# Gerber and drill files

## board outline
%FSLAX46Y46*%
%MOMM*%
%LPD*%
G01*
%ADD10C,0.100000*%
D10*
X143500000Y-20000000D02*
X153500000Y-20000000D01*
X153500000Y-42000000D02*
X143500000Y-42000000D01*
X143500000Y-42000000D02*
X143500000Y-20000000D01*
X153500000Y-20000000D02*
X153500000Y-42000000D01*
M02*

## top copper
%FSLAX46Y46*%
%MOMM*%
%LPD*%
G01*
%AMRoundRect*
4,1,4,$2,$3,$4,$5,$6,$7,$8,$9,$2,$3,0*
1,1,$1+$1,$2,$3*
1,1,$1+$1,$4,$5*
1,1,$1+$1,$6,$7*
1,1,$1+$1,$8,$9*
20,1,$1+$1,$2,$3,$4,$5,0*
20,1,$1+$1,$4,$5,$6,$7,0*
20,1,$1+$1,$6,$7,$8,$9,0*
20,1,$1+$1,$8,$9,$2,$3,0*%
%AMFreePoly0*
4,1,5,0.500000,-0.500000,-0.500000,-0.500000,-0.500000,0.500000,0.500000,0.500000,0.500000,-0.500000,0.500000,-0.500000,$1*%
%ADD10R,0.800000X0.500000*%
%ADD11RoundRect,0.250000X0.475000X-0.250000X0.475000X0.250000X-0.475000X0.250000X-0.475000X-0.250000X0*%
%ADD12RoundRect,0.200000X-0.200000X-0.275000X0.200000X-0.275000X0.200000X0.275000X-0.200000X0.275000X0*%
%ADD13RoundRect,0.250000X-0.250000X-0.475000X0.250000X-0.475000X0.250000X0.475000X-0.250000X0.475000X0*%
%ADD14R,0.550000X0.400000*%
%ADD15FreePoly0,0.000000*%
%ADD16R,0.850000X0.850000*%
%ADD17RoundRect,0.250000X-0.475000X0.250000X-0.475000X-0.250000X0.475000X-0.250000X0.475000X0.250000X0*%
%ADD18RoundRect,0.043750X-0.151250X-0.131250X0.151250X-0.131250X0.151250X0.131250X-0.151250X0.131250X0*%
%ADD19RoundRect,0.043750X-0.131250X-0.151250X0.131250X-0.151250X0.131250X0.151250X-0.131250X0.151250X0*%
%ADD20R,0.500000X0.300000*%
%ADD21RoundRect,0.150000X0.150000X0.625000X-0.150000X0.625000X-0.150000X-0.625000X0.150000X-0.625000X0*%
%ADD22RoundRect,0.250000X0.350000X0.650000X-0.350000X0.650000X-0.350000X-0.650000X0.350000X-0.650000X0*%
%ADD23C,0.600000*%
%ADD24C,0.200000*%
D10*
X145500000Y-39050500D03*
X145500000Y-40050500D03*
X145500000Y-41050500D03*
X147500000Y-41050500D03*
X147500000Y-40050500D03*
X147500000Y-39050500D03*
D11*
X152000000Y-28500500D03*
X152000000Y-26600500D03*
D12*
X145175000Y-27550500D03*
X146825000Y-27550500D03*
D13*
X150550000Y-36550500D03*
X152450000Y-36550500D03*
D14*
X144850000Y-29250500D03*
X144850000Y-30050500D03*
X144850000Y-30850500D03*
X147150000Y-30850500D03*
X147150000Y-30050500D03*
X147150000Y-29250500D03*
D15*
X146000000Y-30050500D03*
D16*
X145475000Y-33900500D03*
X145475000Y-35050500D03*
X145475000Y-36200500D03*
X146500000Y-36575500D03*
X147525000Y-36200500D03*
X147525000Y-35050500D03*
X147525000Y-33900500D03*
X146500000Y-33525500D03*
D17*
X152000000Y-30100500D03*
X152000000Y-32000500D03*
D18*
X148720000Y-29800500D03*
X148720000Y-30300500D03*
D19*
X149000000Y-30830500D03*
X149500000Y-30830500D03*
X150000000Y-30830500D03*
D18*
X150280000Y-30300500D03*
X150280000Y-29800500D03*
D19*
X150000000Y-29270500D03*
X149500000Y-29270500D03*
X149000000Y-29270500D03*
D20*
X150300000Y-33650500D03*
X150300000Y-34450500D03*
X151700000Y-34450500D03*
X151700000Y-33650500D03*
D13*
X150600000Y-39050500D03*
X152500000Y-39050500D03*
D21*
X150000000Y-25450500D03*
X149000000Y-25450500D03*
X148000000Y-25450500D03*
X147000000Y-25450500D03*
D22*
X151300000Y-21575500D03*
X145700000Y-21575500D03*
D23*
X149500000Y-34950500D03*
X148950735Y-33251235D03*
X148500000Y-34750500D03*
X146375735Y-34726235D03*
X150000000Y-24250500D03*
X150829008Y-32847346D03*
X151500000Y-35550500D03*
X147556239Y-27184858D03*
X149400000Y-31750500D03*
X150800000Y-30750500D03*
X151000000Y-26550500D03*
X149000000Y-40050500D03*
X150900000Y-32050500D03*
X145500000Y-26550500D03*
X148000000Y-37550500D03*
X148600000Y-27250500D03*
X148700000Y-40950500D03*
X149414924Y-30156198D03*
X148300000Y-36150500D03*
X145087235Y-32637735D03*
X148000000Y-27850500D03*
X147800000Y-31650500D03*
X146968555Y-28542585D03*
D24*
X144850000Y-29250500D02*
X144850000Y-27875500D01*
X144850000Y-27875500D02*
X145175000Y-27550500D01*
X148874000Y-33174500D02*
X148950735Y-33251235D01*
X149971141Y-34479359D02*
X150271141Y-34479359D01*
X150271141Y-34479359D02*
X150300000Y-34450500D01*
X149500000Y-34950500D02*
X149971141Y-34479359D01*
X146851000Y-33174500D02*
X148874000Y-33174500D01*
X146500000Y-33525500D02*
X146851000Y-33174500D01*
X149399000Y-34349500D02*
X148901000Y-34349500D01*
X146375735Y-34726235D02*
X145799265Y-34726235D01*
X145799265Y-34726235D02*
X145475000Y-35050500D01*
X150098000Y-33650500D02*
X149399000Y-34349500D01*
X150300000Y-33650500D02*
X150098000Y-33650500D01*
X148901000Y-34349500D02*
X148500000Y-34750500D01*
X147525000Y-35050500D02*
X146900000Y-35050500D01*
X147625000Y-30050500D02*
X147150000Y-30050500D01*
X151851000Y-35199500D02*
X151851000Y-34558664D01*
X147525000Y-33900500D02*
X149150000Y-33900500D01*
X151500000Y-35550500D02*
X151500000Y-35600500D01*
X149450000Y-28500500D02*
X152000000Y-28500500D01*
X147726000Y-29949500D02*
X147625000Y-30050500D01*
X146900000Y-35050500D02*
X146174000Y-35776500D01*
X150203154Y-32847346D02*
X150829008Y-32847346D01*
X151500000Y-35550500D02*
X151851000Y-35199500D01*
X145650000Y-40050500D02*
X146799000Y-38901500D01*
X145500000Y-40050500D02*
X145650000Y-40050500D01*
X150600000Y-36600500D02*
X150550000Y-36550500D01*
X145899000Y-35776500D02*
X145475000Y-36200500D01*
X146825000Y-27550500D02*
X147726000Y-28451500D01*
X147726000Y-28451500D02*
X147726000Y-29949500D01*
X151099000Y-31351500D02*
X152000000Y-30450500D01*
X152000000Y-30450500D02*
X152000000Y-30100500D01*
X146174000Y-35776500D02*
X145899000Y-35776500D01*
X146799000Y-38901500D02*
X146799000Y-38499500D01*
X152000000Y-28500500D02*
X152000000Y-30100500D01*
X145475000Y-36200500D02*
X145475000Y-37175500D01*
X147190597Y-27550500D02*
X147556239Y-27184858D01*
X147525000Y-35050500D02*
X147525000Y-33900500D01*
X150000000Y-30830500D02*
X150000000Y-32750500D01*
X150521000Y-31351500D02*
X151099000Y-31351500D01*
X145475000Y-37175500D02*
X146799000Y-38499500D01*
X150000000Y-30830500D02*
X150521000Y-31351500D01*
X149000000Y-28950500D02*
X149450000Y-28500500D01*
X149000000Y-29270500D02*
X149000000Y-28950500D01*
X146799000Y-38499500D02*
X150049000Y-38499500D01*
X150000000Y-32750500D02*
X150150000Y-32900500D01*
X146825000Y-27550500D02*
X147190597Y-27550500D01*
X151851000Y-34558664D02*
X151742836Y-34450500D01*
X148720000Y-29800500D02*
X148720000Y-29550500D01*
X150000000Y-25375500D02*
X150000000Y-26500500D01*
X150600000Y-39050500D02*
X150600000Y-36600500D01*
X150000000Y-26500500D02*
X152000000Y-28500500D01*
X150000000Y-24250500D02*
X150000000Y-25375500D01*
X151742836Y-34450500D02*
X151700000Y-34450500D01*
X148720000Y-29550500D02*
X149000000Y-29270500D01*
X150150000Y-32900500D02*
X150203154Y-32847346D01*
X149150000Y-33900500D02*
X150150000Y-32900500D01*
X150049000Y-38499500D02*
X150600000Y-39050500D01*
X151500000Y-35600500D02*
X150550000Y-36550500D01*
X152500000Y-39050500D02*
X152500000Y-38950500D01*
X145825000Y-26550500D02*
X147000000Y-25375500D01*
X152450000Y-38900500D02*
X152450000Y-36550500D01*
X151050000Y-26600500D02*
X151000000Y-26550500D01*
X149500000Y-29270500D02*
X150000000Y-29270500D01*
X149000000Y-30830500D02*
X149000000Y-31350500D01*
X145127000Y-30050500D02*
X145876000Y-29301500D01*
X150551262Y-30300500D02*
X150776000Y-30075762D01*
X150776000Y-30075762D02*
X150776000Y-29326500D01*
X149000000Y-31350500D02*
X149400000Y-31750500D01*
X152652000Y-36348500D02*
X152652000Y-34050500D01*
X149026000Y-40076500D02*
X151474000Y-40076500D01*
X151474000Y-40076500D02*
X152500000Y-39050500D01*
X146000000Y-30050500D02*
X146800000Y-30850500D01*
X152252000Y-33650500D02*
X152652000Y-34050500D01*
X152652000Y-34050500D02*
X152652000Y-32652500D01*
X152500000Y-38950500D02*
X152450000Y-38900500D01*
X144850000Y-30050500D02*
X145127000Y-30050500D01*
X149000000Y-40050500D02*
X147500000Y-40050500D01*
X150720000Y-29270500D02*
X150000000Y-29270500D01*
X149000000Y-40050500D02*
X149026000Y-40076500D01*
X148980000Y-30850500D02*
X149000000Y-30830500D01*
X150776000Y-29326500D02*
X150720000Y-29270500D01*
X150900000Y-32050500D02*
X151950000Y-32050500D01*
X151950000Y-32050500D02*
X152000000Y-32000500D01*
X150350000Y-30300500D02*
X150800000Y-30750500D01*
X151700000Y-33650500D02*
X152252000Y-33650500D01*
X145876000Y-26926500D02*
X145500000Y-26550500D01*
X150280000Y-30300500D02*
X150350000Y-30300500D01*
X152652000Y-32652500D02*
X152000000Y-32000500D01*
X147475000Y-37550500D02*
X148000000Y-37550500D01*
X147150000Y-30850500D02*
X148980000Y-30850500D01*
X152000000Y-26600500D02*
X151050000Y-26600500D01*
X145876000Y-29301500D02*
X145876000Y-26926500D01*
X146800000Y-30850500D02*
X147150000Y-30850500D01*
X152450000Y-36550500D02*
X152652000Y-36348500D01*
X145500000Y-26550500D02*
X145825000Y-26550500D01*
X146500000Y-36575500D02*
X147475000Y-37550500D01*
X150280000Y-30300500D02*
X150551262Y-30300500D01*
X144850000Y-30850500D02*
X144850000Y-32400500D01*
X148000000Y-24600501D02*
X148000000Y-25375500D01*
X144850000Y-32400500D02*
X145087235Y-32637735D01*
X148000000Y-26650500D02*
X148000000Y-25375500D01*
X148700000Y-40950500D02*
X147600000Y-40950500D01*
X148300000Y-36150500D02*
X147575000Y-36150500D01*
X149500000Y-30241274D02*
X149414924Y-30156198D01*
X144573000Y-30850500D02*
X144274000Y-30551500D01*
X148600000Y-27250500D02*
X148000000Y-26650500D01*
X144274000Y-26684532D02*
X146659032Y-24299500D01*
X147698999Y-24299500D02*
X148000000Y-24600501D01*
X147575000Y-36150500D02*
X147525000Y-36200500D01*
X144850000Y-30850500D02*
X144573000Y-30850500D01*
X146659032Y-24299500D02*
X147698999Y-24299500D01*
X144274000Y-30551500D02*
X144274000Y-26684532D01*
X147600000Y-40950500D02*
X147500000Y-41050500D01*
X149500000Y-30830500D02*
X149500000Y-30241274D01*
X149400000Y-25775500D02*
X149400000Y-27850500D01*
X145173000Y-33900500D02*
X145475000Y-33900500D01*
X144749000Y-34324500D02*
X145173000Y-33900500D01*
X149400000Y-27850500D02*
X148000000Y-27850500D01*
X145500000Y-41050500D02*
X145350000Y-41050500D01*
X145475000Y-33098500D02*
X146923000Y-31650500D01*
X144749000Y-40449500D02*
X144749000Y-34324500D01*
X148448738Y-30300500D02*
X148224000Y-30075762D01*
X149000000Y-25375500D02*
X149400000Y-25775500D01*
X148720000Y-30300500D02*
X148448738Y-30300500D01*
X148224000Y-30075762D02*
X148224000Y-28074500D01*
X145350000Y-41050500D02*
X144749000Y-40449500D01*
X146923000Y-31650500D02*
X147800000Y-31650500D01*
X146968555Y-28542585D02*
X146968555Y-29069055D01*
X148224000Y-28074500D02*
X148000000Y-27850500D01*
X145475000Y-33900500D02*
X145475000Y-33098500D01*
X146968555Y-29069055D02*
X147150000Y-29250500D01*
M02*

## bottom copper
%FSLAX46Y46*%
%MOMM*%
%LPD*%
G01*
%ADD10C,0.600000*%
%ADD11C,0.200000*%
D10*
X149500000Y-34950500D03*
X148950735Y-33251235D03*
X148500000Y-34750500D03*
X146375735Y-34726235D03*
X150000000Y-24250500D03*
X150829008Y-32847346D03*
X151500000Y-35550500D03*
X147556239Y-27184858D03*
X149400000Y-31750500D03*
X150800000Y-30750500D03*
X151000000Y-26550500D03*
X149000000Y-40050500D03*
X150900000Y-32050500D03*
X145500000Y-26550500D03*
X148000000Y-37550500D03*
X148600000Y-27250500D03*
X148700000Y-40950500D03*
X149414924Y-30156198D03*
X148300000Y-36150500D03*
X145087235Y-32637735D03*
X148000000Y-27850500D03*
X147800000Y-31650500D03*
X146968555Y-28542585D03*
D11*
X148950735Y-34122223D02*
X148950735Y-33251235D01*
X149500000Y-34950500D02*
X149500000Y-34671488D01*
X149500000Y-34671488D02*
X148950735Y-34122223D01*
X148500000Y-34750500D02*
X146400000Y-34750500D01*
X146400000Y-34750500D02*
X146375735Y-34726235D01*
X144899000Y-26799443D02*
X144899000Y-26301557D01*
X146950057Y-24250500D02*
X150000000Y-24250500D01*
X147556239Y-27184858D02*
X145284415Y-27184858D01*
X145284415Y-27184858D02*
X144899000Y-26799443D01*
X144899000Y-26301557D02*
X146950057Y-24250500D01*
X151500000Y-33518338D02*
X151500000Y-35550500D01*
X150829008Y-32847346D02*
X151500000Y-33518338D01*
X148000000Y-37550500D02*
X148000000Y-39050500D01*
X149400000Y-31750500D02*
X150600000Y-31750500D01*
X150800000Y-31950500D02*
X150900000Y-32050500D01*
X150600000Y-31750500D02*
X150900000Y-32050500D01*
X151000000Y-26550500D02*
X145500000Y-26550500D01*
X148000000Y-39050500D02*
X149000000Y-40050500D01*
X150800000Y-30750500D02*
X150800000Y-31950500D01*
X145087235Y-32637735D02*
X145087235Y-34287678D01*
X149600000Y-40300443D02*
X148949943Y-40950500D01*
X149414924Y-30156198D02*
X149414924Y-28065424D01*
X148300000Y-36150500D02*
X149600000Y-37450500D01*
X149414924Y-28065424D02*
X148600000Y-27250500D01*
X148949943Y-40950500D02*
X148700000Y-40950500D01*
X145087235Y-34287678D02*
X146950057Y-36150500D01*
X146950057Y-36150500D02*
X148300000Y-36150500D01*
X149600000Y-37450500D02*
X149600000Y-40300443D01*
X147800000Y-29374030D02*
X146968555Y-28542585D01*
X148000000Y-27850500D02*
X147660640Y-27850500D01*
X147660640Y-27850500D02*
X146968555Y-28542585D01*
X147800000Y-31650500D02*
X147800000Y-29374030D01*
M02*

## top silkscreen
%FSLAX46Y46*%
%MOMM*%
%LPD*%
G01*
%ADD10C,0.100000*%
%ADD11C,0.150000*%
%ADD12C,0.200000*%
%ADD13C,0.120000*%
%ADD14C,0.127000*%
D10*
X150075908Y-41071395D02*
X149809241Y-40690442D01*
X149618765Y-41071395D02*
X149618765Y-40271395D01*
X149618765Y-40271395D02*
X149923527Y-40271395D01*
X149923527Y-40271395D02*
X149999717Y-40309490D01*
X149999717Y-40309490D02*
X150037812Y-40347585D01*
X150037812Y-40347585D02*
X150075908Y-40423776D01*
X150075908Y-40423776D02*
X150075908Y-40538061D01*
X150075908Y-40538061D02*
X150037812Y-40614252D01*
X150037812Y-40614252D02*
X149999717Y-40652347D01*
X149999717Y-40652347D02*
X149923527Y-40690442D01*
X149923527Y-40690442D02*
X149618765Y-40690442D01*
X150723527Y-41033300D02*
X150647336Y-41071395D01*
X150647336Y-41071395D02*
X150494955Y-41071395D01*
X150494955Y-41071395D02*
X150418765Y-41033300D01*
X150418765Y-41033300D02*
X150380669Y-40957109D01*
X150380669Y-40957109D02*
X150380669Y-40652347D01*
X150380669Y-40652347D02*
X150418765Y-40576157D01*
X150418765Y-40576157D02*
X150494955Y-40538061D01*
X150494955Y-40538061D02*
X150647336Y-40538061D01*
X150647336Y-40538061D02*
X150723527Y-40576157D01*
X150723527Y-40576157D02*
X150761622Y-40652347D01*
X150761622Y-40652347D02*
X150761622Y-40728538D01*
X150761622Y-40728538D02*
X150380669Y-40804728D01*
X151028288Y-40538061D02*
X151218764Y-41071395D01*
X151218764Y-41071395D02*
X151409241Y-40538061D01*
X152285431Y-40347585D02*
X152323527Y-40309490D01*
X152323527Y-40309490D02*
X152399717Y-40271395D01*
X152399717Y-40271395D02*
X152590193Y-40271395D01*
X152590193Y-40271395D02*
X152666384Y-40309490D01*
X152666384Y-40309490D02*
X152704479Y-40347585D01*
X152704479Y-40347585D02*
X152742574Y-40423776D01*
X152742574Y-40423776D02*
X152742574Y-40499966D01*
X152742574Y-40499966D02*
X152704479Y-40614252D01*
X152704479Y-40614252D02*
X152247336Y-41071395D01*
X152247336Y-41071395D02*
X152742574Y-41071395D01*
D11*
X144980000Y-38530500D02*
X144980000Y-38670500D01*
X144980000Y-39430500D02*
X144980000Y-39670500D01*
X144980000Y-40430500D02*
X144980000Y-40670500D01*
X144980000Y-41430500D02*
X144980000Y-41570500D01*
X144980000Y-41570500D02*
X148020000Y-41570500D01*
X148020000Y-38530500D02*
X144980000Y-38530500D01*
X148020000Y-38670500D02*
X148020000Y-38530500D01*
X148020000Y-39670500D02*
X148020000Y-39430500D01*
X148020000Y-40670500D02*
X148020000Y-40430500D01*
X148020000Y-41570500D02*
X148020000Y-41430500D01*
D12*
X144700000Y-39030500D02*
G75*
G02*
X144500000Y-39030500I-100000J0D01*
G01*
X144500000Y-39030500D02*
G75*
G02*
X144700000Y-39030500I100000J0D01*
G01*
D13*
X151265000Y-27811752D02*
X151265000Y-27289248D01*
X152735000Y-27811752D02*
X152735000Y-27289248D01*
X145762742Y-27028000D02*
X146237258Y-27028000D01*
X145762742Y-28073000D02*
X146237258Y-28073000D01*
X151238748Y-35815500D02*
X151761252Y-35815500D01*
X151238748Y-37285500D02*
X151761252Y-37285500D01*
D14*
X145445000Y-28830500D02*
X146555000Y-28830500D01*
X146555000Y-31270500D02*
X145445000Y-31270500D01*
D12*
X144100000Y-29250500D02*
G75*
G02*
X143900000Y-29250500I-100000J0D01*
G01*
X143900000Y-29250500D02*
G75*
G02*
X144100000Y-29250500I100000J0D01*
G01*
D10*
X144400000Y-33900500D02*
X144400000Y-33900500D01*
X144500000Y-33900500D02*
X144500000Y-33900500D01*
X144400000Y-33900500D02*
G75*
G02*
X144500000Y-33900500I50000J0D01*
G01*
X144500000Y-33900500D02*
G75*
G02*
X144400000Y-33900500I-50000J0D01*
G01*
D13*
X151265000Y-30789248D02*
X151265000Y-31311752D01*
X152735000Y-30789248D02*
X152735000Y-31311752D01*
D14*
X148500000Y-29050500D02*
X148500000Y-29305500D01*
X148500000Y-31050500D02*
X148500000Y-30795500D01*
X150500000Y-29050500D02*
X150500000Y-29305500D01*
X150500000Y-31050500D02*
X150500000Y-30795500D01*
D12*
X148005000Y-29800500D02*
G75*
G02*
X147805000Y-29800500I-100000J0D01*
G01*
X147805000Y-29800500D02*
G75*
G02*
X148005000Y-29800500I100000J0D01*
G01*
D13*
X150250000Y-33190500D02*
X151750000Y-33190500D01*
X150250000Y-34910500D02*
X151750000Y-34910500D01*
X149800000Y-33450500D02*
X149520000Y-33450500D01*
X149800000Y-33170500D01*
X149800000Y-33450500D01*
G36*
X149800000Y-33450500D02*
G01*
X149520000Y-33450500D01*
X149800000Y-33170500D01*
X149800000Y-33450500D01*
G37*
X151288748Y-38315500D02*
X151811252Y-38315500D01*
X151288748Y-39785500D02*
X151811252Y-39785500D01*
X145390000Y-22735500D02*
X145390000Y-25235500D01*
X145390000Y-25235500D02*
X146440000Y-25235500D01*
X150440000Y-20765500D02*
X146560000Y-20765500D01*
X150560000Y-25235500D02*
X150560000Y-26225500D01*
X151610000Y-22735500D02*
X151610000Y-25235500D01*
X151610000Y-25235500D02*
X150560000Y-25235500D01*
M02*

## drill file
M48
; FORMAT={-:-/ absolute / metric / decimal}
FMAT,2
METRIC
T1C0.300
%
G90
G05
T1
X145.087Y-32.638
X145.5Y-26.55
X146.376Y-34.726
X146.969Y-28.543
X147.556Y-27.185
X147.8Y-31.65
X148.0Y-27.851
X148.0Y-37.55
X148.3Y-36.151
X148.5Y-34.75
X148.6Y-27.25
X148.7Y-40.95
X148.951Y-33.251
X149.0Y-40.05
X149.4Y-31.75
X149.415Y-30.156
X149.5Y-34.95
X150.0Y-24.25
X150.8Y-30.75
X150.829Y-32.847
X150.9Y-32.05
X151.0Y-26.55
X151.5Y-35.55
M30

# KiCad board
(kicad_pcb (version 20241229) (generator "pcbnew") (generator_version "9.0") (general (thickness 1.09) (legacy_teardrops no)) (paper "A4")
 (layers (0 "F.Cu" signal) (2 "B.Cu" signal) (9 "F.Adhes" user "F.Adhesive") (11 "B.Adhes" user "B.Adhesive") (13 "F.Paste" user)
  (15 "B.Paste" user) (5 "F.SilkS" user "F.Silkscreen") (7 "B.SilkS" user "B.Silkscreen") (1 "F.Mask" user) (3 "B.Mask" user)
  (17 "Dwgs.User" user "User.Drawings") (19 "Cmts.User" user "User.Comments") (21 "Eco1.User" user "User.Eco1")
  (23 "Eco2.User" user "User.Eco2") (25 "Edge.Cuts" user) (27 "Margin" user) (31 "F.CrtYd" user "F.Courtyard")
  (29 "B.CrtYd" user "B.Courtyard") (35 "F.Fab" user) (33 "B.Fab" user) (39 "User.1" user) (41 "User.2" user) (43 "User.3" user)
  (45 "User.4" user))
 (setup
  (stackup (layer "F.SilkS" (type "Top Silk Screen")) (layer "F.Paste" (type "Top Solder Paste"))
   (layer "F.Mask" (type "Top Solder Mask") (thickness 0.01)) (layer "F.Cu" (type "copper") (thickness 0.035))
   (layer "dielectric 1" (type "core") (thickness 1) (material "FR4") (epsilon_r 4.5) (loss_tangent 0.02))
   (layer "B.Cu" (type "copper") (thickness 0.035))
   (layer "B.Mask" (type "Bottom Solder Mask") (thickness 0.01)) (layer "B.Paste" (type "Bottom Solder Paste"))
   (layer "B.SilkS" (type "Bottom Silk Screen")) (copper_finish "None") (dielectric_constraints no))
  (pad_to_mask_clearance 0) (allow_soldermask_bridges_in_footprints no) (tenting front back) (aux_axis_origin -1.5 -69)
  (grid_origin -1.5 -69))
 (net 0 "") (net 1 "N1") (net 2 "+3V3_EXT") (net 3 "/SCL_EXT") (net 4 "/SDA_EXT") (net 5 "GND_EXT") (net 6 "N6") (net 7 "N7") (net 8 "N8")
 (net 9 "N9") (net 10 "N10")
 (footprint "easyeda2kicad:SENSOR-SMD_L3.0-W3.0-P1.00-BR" (layer "F.Cu") (at 146.5 40.0505 180)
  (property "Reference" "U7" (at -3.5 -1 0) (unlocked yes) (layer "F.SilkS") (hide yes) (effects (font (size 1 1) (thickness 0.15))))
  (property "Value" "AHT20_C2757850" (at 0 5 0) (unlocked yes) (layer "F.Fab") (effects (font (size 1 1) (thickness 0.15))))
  (fp_line (start 1.52 1.52) (end 1.52 1.38) (stroke (width 0.15) (type solid)) (layer "F.SilkS"))
  (fp_line (start 1.52 0.62) (end 1.52 0.38) (stroke (width 0.15) (type solid)) (layer "F.SilkS"))
  (fp_line (start 1.52 -0.38) (end 1.52 -0.62) (stroke (width 0.15) (type solid)) (layer "F.SilkS"))
  (fp_line (start 1.52 -1.38) (end 1.52 -1.52) (stroke (width 0.15) (type solid)) (layer "F.SilkS"))
  (fp_line (start 1.52 -1.52) (end -1.52 -1.52) (stroke (width 0.15) (type solid)) (layer "F.SilkS"))
  (fp_line (start -1.52 1.52) (end 1.52 1.52) (stroke (width 0.15) (type solid)) (layer "F.SilkS"))
  (fp_line (start -1.52 1.38) (end -1.52 1.52) (stroke (width 0.15) (type solid)) (layer "F.SilkS"))
  (fp_line (start -1.52 0.38) (end -1.52 0.62) (stroke (width 0.15) (type solid)) (layer "F.SilkS"))
  (fp_line (start -1.52 -0.62) (end -1.52 -0.38) (stroke (width 0.15) (type solid)) (layer "F.SilkS"))
  (fp_line (start -1.52 -1.52) (end -1.52 -1.38) (stroke (width 0.15) (type solid)) (layer "F.SilkS"))
  (fp_circle (center 1.9 1.02) (end 2 1.02) (stroke (width 0.2) (type solid)) (fill no) (layer "F.SilkS"))
  (pad "1" smd rect (at 1 1) (size 0.8 0.5) (layers "F.Cu" "F.Mask" "F.Paste") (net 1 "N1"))
  (pad "2" smd rect (at 1 0) (size 0.8 0.5) (layers "F.Cu" "F.Mask" "F.Paste") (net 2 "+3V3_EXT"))
  (pad "3" smd rect (at 1 -1) (size 0.8 0.5) (layers "F.Cu" "F.Mask" "F.Paste") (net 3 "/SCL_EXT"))
  (pad "4" smd rect (at -1 -1) (size 0.8 0.5) (layers "F.Cu" "F.Mask" "F.Paste") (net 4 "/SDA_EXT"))
  (pad "5" smd rect (at -1 0) (size 0.8 0.5) (layers "F.Cu" "F.Mask" "F.Paste") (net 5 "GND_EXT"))
  (pad "6" smd rect (at -1 1) (size 0.8 0.5) (layers "F.Cu" "F.Mask" "F.Paste") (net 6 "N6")))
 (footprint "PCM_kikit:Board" (layer "F.Cu") (at 143.5 20)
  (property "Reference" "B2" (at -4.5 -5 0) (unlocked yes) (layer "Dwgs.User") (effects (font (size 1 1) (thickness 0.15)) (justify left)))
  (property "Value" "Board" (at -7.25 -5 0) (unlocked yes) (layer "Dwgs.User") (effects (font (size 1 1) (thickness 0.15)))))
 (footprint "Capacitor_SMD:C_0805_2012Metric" (layer "F.Cu") (at 152 27.5505 90)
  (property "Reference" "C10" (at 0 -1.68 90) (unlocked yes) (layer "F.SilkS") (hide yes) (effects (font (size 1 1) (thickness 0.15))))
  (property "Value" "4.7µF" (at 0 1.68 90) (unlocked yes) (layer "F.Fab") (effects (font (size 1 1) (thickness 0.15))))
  (fp_line (start -0.261252 -0.735) (end 0.261252 -0.735) (stroke (width 0.12) (type solid)) (layer "F.SilkS"))
  (fp_line (start -0.261252 0.735) (end 0.261252 0.735) (stroke (width 0.12) (type solid)) (layer "F.SilkS"))
  (pad "1" smd roundrect (at -0.95 0 90) (size 1 1.45) (layers "F.Cu" "F.Mask" "F.Paste") (roundrect_rratio 0.25) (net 2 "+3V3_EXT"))
  (pad "2" smd roundrect (at 0.95 0 90) (size 1 1.45) (layers "F.Cu" "F.Mask" "F.Paste") (roundrect_rratio 0.25) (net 5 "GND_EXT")))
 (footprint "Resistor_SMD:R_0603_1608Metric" (layer "F.Cu") (at 146 27.5505)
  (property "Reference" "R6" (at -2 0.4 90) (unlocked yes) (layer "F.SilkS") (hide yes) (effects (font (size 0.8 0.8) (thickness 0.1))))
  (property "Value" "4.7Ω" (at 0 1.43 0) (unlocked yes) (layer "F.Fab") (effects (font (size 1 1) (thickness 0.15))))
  (fp_line (start -0.237258 -0.5225) (end 0.237258 -0.5225) (stroke (width 0.12) (type solid)) (layer "F.SilkS"))
  (fp_line (start -0.237258 0.5225) (end 0.237258 0.5225) (stroke (width 0.12) (type solid)) (layer "F.SilkS"))
  (pad "1" smd roundrect (at -0.825 0) (size 0.8 0.95) (layers "F.Cu" "F.Mask" "F.Paste") (roundrect_rratio 0.25) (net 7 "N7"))
  (pad "2" smd roundrect (at 0.825 0) (size 0.8 0.95) (layers "F.Cu" "F.Mask" "F.Paste") (roundrect_rratio 0.25) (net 2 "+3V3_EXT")))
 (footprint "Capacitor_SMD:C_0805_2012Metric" (layer "F.Cu") (at 151.5 36.5505)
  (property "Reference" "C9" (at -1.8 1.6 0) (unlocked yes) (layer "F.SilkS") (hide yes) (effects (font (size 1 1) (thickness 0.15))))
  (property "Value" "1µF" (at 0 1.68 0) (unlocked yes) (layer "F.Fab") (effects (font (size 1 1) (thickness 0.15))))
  (fp_line (start -0.261252 -0.735) (end 0.261252 -0.735) (stroke (width 0.12) (type solid)) (layer "F.SilkS"))
  (fp_line (start -0.261252 0.735) (end 0.261252 0.735) (stroke (width 0.12) (type solid)) (layer "F.SilkS"))
  (pad "1" smd roundrect (at -0.95 0) (size 1 1.45) (layers "F.Cu" "F.Mask" "F.Paste") (roundrect_rratio 0.25) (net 2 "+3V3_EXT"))
  (pad "2" smd roundrect (at 0.95 0) (size 1 1.45) (layers "F.Cu" "F.Mask" "F.Paste") (roundrect_rratio 0.25) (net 5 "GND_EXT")))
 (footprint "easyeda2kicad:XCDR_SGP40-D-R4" (layer "F.Cu") (at 146 30.0505)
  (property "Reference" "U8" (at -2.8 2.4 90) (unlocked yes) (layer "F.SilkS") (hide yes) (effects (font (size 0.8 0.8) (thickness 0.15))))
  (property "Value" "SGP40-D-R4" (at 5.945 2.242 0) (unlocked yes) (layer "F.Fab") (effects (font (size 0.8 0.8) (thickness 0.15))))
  (fp_line (start -0.555 -1.22) (end 0.555 -1.22) (stroke (width 0.127) (type solid)) (layer "F.SilkS"))
  (fp_line (start 0.555 1.22) (end -0.555 1.22) (stroke (width 0.127) (type solid)) (layer "F.SilkS"))
  (fp_circle (center -2 -0.8) (end -1.9 -0.8) (stroke (width 0.2) (type solid)) (fill no) (layer "F.SilkS"))
  (pad "1" smd rect (at -1.15 -0.8) (size 0.55 0.4) (layers "F.Cu" "F.Mask" "F.Paste") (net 7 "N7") (solder_mask_margin 0.102))
  (pad "2" smd rect (at -1.15 0) (size 0.55 0.4) (layers "F.Cu" "F.Mask" "F.Paste") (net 5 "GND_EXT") (solder_mask_margin 0.102))
  (pad "3" smd rect (at -1.15 0.8) (size 0.55 0.4) (layers "F.Cu" "F.Mask" "F.Paste") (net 4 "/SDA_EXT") (solder_mask_margin 0.102))
  (pad "4" smd rect (at 1.15 0.8) (size 0.55 0.4) (layers "F.Cu" "F.Mask" "F.Paste") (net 5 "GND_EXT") (solder_mask_margin 0.102))
  (pad "5" smd rect (at 1.15 0) (size 0.55 0.4) (layers "F.Cu" "F.Mask" "F.Paste") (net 2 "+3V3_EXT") (solder_mask_margin 0.102))
  (pad "6" smd rect (at 1.15 -0.8) (size 0.55 0.4) (layers "F.Cu" "F.Mask" "F.Paste") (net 3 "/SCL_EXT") (solder_mask_margin 0.102))
  (pad "7" smd custom (at 0 0) (size 1 1) (layers "F.Cu") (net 5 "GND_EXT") (options (clearance outline) (anchor rect)) (primitives)))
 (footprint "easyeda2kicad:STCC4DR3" (layer "F.Cu") (at 146.5 35.0505)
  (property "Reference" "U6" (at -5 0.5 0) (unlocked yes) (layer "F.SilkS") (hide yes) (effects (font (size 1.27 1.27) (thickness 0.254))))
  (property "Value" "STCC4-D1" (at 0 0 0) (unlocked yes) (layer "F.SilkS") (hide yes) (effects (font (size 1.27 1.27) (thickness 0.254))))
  (fp_line (start -2.1 -1.15) (end -2.1 -1.15) (stroke (width 0.1) (type solid)) (layer "F.SilkS"))
  (fp_line (start -2 -1.15) (end -2 -1.15) (stroke (width 0.1) (type solid)) (layer "F.SilkS"))
  (fp_arc (start -2.1 -1.15) (mid -2.05 -1.2) (end -2 -1.15) (stroke (width 0.1) (type solid)) (layer "F.SilkS"))
  (fp_arc (start -2 -1.15) (mid -2.05 -1.1) (end -2.1 -1.15) (stroke (width 0.1) (type solid)) (layer "F.SilkS"))
  (pad "1" smd rect (at -1.025 -1.15 90) (size 0.85 0.85) (layers "F.Cu" "F.Mask" "F.Paste") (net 3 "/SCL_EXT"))
  (pad "2" smd rect (at -1.025 0 90) (size 0.85 0.85) (layers "F.Cu" "F.Mask" "F.Paste") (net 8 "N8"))
  (pad "3" smd rect (at -1.025 1.15 90) (size 0.85 0.85) (layers "F.Cu" "F.Mask" "F.Paste") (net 2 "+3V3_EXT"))
  (pad "4" smd rect (at 0 1.525 90) (size 0.85 0.85) (layers "F.Cu" "F.Mask" "F.Paste") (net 5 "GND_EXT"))
  (pad "5" smd rect (at 1.025 1.15 90) (size 0.85 0.85) (layers "F.Cu" "F.Mask" "F.Paste") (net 4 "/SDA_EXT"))
  (pad "6" smd rect (at 1.025 0 90) (size 0.85 0.85) (layers "F.Cu" "F.Mask" "F.Paste") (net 2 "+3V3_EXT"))
  (pad "7" smd rect (at 1.025 -1.15 90) (size 0.85 0.85) (layers "F.Cu" "F.Mask" "F.Paste") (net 2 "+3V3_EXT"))
  (pad "8" smd rect (at 0 -1.525 90) (size 0.85 0.85) (layers "F.Cu" "F.Mask" "F.Paste") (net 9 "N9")))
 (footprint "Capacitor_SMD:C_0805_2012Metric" (layer "F.Cu") (at 152 31.0505 -90)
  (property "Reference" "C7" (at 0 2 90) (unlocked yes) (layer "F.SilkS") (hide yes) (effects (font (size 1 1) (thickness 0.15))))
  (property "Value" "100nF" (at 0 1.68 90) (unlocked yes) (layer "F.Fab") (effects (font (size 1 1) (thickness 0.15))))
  (fp_line (start -0.261252 0.735) (end 0.261252 0.735) (stroke (width 0.12) (type solid)) (layer "F.SilkS"))
  (fp_line (start -0.261252 -0.735) (end 0.261252 -0.735) (stroke (width 0.12) (type solid)) (layer "F.SilkS"))
  (pad "1" smd roundrect (at -0.95 0 270) (size 1 1.45) (layers "F.Cu" "F.Mask" "F.Paste") (roundrect_rratio 0.25) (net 2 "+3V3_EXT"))
  (pad "2" smd roundrect (at 0.95 0 270) (size 1 1.45) (layers "F.Cu" "F.Mask" "F.Paste") (roundrect_rratio 0.25) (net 5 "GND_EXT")))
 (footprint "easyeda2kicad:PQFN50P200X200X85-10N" (layer "F.Cu") (at 149.5 30.0505)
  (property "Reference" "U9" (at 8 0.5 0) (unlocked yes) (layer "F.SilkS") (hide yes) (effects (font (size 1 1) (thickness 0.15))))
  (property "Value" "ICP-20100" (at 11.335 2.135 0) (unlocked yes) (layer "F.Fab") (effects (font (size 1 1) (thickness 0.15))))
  (fp_line (start -1 -1) (end -1 -0.745) (stroke (width 0.127) (type solid)) (layer "F.SilkS"))
  (fp_line (start -1 1) (end -1 0.745) (stroke (width 0.127) (type solid)) (layer "F.SilkS"))
  (fp_line (start 1 -1) (end 1 -0.745) (stroke (width 0.127) (type solid)) (layer "F.SilkS"))
  (fp_line (start 1 1) (end 1 0.745) (stroke (width 0.127) (type solid)) (layer "F.SilkS"))
  (fp_circle (center -1.595 -0.25) (end -1.495 -0.25) (stroke (width 0.2) (type solid)) (fill no) (layer "F.SilkS"))
  (pad "1" smd roundrect (at -0.78 -0.25) (size 0.39 0.35) (layers "F.Cu" "F.Mask" "F.Paste") (roundrect_rratio 0.125) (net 2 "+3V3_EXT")
   (solder_mask_margin 0.102))
  (pad "2" smd roundrect (at -0.78 0.25) (size 0.39 0.35) (layers "F.Cu" "F.Mask" "F.Paste") (roundrect_rratio 0.125) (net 3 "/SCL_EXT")
   (solder_mask_margin 0.102))
  (pad "3" smd roundrect (at -0.5 0.78) (size 0.35 0.39) (layers "F.Cu" "F.Mask" "F.Paste") (roundrect_rratio 0.125) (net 5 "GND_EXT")
   (solder_mask_margin 0.102))
  (pad "4" smd roundrect (at 0 0.78) (size 0.35 0.39) (layers "F.Cu" "F.Mask" "F.Paste") (roundrect_rratio 0.125) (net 4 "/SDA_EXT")
   (solder_mask_margin 0.102))
  (pad "5" smd roundrect (at 0.5 0.78) (size 0.35 0.39) (layers "F.Cu" "F.Mask" "F.Paste") (roundrect_rratio 0.125) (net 2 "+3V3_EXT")
   (solder_mask_margin 0.102))
  (pad "6" smd roundrect (at 0.78 0.25) (size 0.39 0.35) (layers "F.Cu" "F.Mask" "F.Paste") (roundrect_rratio 0.125) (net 5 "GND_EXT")
   (solder_mask_margin 0.102))
  (pad "7" smd roundrect (at 0.78 -0.25) (size 0.39 0.35) (layers "F.Cu" "F.Mask" "F.Paste") (roundrect_rratio 0.125) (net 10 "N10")
   (solder_mask_margin 0.102))
  (pad "8" smd roundrect (at 0.5 -0.78) (size 0.35 0.39) (layers "F.Cu" "F.Mask" "F.Paste") (roundrect_rratio 0.125) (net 5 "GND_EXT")
   (solder_mask_margin 0.102))
  (pad "9" smd roundrect (at 0 -0.78) (size 0.35 0.39) (layers "F.Cu" "F.Mask" "F.Paste") (roundrect_rratio 0.125) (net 5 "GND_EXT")
   (solder_mask_margin 0.102))
  (pad "10" smd roundrect (at -0.5 -0.78) (size 0.35 0.39) (layers "F.Cu" "F.Mask" "F.Paste") (roundrect_rratio 0.125) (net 2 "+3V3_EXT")
   (solder_mask_margin 0.102)))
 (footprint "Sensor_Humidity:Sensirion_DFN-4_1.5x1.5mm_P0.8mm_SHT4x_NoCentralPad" (layer "F.Cu") (at 151 34.0505)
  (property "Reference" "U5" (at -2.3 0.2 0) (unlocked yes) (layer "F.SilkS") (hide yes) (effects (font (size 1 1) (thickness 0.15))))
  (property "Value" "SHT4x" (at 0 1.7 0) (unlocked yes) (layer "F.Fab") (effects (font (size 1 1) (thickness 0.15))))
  (fp_line (start -0.75 -0.86) (end 0.75 -0.86) (stroke (width 0.12) (type solid)) (layer "F.SilkS"))
  (fp_line (start -0.75 0.86) (end 0.75 0.86) (stroke (width 0.12) (type solid)) (layer "F.SilkS"))
  (fp_poly
   (pts (xy -1.2 -0.6) (xy -1.48 -0.6) (xy -1.2 -0.88) (xy -1.2 -0.6)) (stroke (width 0.12) (type solid)) (fill yes) (layer "F.SilkS"))
  (pad "1" smd rect (at -0.7 -0.4) (size 0.5 0.3) (layers "F.Cu" "F.Mask" "F.Paste") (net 8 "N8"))
  (pad "2" smd rect (at -0.7 0.4) (size 0.5 0.3) (layers "F.Cu" "F.Mask" "F.Paste") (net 9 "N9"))
  (pad "3" smd rect (at 0.7 0.4) (size 0.5 0.3) (layers "F.Cu" "F.Mask" "F.Paste") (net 2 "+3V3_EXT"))
  (pad "4" smd rect (at 0.7 -0.4) (size 0.5 0.3) (layers "F.Cu" "F.Mask" "F.Paste") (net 5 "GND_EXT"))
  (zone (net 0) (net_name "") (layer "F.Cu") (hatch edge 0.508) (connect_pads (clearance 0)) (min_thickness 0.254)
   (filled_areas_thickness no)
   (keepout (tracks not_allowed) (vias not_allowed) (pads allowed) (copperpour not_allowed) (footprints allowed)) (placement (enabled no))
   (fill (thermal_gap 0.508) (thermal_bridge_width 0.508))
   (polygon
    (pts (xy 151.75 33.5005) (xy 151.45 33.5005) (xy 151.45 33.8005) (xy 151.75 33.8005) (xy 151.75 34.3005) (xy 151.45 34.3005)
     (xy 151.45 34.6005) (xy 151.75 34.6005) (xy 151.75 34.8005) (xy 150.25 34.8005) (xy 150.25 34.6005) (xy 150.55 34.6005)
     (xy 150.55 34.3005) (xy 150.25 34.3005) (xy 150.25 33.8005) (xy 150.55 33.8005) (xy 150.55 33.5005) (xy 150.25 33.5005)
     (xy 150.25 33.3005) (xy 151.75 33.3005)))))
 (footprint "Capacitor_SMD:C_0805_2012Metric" (layer "F.Cu") (at 151.55 39.0505)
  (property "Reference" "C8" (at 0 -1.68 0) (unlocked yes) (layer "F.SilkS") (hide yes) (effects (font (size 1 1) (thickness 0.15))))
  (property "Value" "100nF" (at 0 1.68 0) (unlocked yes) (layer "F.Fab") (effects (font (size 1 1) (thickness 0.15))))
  (fp_line (start -0.261252 -0.735) (end 0.261252 -0.735) (stroke (width 0.12) (type solid)) (layer "F.SilkS"))
  (fp_line (start -0.261252 0.735) (end 0.261252 0.735) (stroke (width 0.12) (type solid)) (layer "F.SilkS"))
  (pad "1" smd roundrect (at -0.95 0) (size 1 1.45) (layers "F.Cu" "F.Mask" "F.Paste") (roundrect_rratio 0.25) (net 2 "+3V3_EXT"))
  (pad "2" smd roundrect (at 0.95 0) (size 1 1.45) (layers "F.Cu" "F.Mask" "F.Paste") (roundrect_rratio 0.25) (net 5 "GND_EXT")))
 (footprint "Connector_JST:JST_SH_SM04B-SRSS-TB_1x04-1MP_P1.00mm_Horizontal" (layer "F.Cu") (at 148.5 23.4505 180)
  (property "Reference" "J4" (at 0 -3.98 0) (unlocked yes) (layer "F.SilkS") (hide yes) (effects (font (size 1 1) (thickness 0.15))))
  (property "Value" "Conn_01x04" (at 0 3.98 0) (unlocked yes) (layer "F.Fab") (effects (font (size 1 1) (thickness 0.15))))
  (fp_line (start 3.11 0.715) (end 3.11 -1.785) (stroke (width 0.12) (type solid)) (layer "F.SilkS"))
  (fp_line (start 3.11 -1.785) (end 2.06 -1.785) (stroke (width 0.12) (type solid)) (layer "F.SilkS"))
  (fp_line (start -1.94 2.685) (end 1.94 2.685) (stroke (width 0.12) (type solid)) (layer "F.SilkS"))
  (fp_line (start -2.06 -1.785) (end -2.06 -2.775) (stroke (width 0.12) (type solid)) (layer "F.SilkS"))
  (fp_line (start -3.11 0.715) (end -3.11 -1.785) (stroke (width 0.12) (type solid)) (layer "F.SilkS"))
  (fp_line (start -3.11 -1.785) (end -2.06 -1.785) (stroke (width 0.12) (type solid)) (layer "F.SilkS"))
  (pad "1" smd roundrect (at -1.5 -2 180) (size 0.6 1.55) (layers "F.Cu" "F.Mask" "F.Paste") (roundrect_rratio 0.25) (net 2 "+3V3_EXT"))
  (pad "2" smd roundrect (at -0.5 -2 180) (size 0.6 1.55) (layers "F.Cu" "F.Mask" "F.Paste") (roundrect_rratio 0.25) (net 3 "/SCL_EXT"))
  (pad "3" smd roundrect (at 0.5 -2 180) (size 0.6 1.55) (layers "F.Cu" "F.Mask" "F.Paste") (roundrect_rratio 0.25) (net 4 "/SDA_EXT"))
  (pad "4" smd roundrect (at 1.5 -2 180) (size 0.6 1.55) (layers "F.Cu" "F.Mask" "F.Paste") (roundrect_rratio 0.25) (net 5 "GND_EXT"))
  (pad "MP" smd roundrect (at -2.8 1.875 180) (size 1.2 1.8) (layers "F.Cu" "F.Mask" "F.Paste") (roundrect_rratio 0.208333))
  (pad "MP" smd roundrect (at 2.8 1.875 180) (size 1.2 1.8) (layers "F.Cu" "F.Mask" "F.Paste") (roundrect_rratio 0.208333)))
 (gr_line (start 143.5 20) (end 153.5 20) (stroke (width 0.1) (type default)) (layer "Edge.Cuts"))
 (gr_line (start 153.5 42) (end 143.5 42) (stroke (width 0.1) (type default)) (layer "Edge.Cuts"))
 (gr_line (start 143.5 42) (end 143.5 20) (stroke (width 0.1) (type default)) (layer "Edge.Cuts"))
 (gr_line (start 153.5 20) (end 153.5 42) (stroke (width 0.1) (type default)) (layer "Edge.Cuts"))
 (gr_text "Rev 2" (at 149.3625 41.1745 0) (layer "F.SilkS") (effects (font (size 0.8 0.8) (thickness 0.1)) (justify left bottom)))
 (segment (start 144.85 29.2505) (end 144.85 27.8755) (width 0.2) (layer "F.Cu") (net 7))
 (segment (start 144.85 27.8755) (end 145.175 27.5505) (width 0.2) (layer "F.Cu") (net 7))
 (segment (start 148.874 33.1745) (end 148.950735 33.251235) (width 0.2) (layer "F.Cu") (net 9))
 (segment (start 149.971141 34.479359) (end 150.271141 34.479359) (width 0.2) (layer "F.Cu") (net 9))
 (segment (start 150.271141 34.479359) (end 150.3 34.4505) (width 0.2) (layer "F.Cu") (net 9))
 (segment (start 149.5 34.9505) (end 149.971141 34.479359) (width 0.2) (layer "F.Cu") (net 9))
 (segment (start 146.851 33.1745) (end 148.874 33.1745) (width 0.2) (layer "F.Cu") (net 9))
 (segment (start 146.5 33.5255) (end 146.851 33.1745) (width 0.2) (layer "F.Cu") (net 9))
 (via (at 149.5 34.9505) (size 0.6) (drill 0.3) (layers "F.Cu" "B.Cu") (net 9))
 (via (at 148.950735 33.251235) (size 0.6) (drill 0.3) (layers "F.Cu" "B.Cu") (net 9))
 (segment (start 148.950735 34.122223) (end 148.950735 33.251235) (width 0.2) (layer "B.Cu") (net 9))
 (segment (start 149.5 34.9505) (end 149.5 34.671488) (width 0.2) (layer "B.Cu") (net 9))
 (segment (start 149.5 34.671488) (end 148.950735 34.122223) (width 0.2) (layer "B.Cu") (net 9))
 (segment (start 149.399 34.3495) (end 148.901 34.3495) (width 0.2) (layer "F.Cu") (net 8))
 (segment (start 146.375735 34.726235) (end 145.799265 34.726235) (width 0.2) (layer "F.Cu") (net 8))
 (segment (start 145.799265 34.726235) (end 145.475 35.0505) (width 0.2) (layer "F.Cu") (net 8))
 (segment (start 150.098 33.6505) (end 149.399 34.3495) (width 0.2) (layer "F.Cu") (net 8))
 (segment (start 150.3 33.6505) (end 150.098 33.6505) (width 0.2) (layer "F.Cu") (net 8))
 (segment (start 148.901 34.3495) (end 148.5 34.7505) (width 0.2) (layer "F.Cu") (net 8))
 (via (at 148.5 34.7505) (size 0.6) (drill 0.3) (layers "F.Cu" "B.Cu") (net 8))
 (via (at 146.375735 34.726235) (size 0.6) (drill 0.3) (layers "F.Cu" "B.Cu") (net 8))
 (segment (start 148.5 34.7505) (end 146.4 34.7505) (width 0.2) (layer "B.Cu") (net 8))
 (segment (start 146.4 34.7505) (end 146.375735 34.726235) (width 0.2) (layer "B.Cu") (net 8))
 (segment (start 147.525 35.0505) (end 146.9 35.0505) (width 0.2) (layer "F.Cu") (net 2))
 (segment (start 147.625 30.0505) (end 147.15 30.0505) (width 0.2) (layer "F.Cu") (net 2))
 (segment (start 151.851 35.1995) (end 151.851 34.558664) (width 0.2) (layer "F.Cu") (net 2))
 (segment (start 147.525 33.9005) (end 149.15 33.9005) (width 0.2) (layer "F.Cu") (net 2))
 (segment (start 151.5 35.5505) (end 151.5 35.6005) (width 0.2) (layer "F.Cu") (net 2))
 (segment (start 149.45 28.5005) (end 152 28.5005) (width 0.2) (layer "F.Cu") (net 2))
 (segment (start 147.726 29.9495) (end 147.625 30.0505) (width 0.2) (layer "F.Cu") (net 2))
 (segment (start 146.9 35.0505) (end 146.174 35.7765) (width 0.2) (layer "F.Cu") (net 2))
 (segment (start 150.203154 32.847346) (end 150.829008 32.847346) (width 0.2) (layer "F.Cu") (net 2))
 (segment (start 151.5 35.5505) (end 151.851 35.1995) (width 0.2) (layer "F.Cu") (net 2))
 (segment (start 145.65 40.0505) (end 146.799 38.9015) (width 0.2) (layer "F.Cu") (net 2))
 (segment (start 145.5 40.0505) (end 145.65 40.0505) (width 0.2) (layer "F.Cu") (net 2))
 (segment (start 150.6 36.6005) (end 150.55 36.5505) (width 0.2) (layer "F.Cu") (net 2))
 (segment (start 145.899 35.7765) (end 145.475 36.2005) (width 0.2) (layer "F.Cu") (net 2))
 (segment (start 146.825 27.5505) (end 147.726 28.4515) (width 0.2) (layer "F.Cu") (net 2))
 (segment (start 147.726 28.4515) (end 147.726 29.9495) (width 0.2) (layer "F.Cu") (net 2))
 (segment (start 151.099 31.3515) (end 152 30.4505) (width 0.2) (layer "F.Cu") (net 2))
 (segment (start 152 30.4505) (end 152 30.1005) (width 0.2) (layer "F.Cu") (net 2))
 (segment (start 146.174 35.7765) (end 145.899 35.7765) (width 0.2) (layer "F.Cu") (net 2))
 (segment (start 146.799 38.9015) (end 146.799 38.4995) (width 0.2) (layer "F.Cu") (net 2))
 (segment (start 152 28.5005) (end 152 30.1005) (width 0.2) (layer "F.Cu") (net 2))
 (segment (start 145.475 36.2005) (end 145.475 37.1755) (width 0.2) (layer "F.Cu") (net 2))
 (segment (start 147.190597 27.5505) (end 147.556239 27.184858) (width 0.2) (layer "F.Cu") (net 2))
 (segment (start 147.525 35.0505) (end 147.525 33.9005) (width 0.2) (layer "F.Cu") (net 2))
 (segment (start 150 30.8305) (end 150 32.7505) (width 0.2) (layer "F.Cu") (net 2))
 (segment (start 150.521 31.3515) (end 151.099 31.3515) (width 0.2) (layer "F.Cu") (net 2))
 (segment (start 145.475 37.1755) (end 146.799 38.4995) (width 0.2) (layer "F.Cu") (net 2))
 (segment (start 150 30.8305) (end 150.521 31.3515) (width 0.2) (layer "F.Cu") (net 2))
 (segment (start 149 28.9505) (end 149.45 28.5005) (width 0.2) (layer "F.Cu") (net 2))
 (segment (start 149 29.2705) (end 149 28.9505) (width 0.2) (layer "F.Cu") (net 2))
 (segment (start 146.799 38.4995) (end 150.049 38.4995) (width 0.2) (layer "F.Cu") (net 2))
 (segment (start 150 32.7505) (end 150.15 32.9005) (width 0.2) (layer "F.Cu") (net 2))
 (segment (start 146.825 27.5505) (end 147.190597 27.5505) (width 0.2) (layer "F.Cu") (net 2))
 (segment (start 151.851 34.558664) (end 151.742836 34.4505) (width 0.2) (layer "F.Cu") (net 2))
 (segment (start 148.72 29.8005) (end 148.72 29.5505) (width 0.2) (layer "F.Cu") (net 2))
 (segment (start 150 25.3755) (end 150 26.5005) (width 0.2) (layer "F.Cu") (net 2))
 (segment (start 150.6 39.0505) (end 150.6 36.6005) (width 0.2) (layer "F.Cu") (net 2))
 (segment (start 150 26.5005) (end 152 28.5005) (width 0.2) (layer "F.Cu") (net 2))
 (segment (start 150 24.2505) (end 150 25.3755) (width 0.2) (layer "F.Cu") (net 2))
 (segment (start 151.742836 34.4505) (end 151.7 34.4505) (width 0.2) (layer "F.Cu") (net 2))
 (segment (start 148.72 29.5505) (end 149 29.2705) (width 0.2) (layer "F.Cu") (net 2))
 (segment (start 150.15 32.9005) (end 150.203154 32.847346) (width 0.2) (layer "F.Cu") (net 2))
 (segment (start 149.15 33.9005) (end 150.15 32.9005) (width 0.2) (layer "F.Cu") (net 2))
 (segment (start 150.049 38.4995) (end 150.6 39.0505) (width 0.2) (layer "F.Cu") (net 2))
 (segment (start 151.5 35.6005) (end 150.55 36.5505) (width 0.2) (layer "F.Cu") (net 2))
 (via (at 150 24.2505) (size 0.6) (drill 0.3) (layers "F.Cu" "B.Cu") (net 2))
 (via (at 150.829008 32.847346) (size 0.6) (drill 0.3) (layers "F.Cu" "B.Cu") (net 2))
 (via (at 151.5 35.5505) (size 0.6) (drill 0.3) (layers "F.Cu" "B.Cu") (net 2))
 (via (at 147.556239 27.184858) (size 0.6) (drill 0.3) (layers "F.Cu" "B.Cu") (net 2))
 (segment (start 144.899 26.799443) (end 144.899 26.301557) (width 0.2) (layer "B.Cu") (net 2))
 (segment (start 146.950057 24.2505) (end 150 24.2505) (width 0.2) (layer "B.Cu") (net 2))
 (segment (start 147.556239 27.184858) (end 145.284415 27.184858) (width 0.2) (layer "B.Cu") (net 2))
 (segment (start 145.284415 27.184858) (end 144.899 26.799443) (width 0.2) (layer "B.Cu") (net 2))
 (segment (start 144.899 26.301557) (end 146.950057 24.2505) (width 0.2) (layer "B.Cu") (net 2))
 (segment (start 151.5 33.518338) (end 151.5 35.5505) (width 0.2) (layer "B.Cu") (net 2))
 (segment (start 150.829008 32.847346) (end 151.5 33.518338) (width 0.2) (layer "B.Cu") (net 2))
 (segment (start 152.5 39.0505) (end 152.5 38.9505) (width 0.2) (layer "F.Cu") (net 5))
 (segment (start 145.825 26.5505) (end 147 25.3755) (width 0.2) (layer "F.Cu") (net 5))
 (segment (start 152.45 38.9005) (end 152.45 36.5505) (width 0.2) (layer "F.Cu") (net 5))
 (segment (start 151.05 26.6005) (end 151 26.5505) (width 0.2) (layer "F.Cu") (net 5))
 (segment (start 149.5 29.2705) (end 150 29.2705) (width 0.2) (layer "F.Cu") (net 5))
 (segment (start 149 30.8305) (end 149 31.3505) (width 0.2) (layer "F.Cu") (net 5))
 (segment (start 145.127 30.0505) (end 145.876 29.3015) (width 0.2) (layer "F.Cu") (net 5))
 (segment (start 150.551262 30.3005) (end 150.776 30.075762) (width 0.2) (layer "F.Cu") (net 5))
 (segment (start 150.776 30.075762) (end 150.776 29.3265) (width 0.2) (layer "F.Cu") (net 5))
 (segment (start 149 31.3505) (end 149.4 31.7505) (width 0.2) (layer "F.Cu") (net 5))
 (segment (start 152.652 36.3485) (end 152.652 34.0505) (width 0.2) (layer "F.Cu") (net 5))
 (segment (start 149.026 40.0765) (end 151.474 40.0765) (width 0.2) (layer "F.Cu") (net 5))
 (segment (start 151.474 40.0765) (end 152.5 39.0505) (width 0.2) (layer "F.Cu") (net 5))
 (segment (start 146 30.0505) (end 146.8 30.8505) (width 0.2) (layer "F.Cu") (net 5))
 (segment (start 152.252 33.6505) (end 152.652 34.0505) (width 0.2) (layer "F.Cu") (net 5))
 (segment (start 152.652 34.0505) (end 152.652 32.6525) (width 0.2) (layer "F.Cu") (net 5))
 (segment (start 152.5 38.9505) (end 152.45 38.9005) (width 0.2) (layer "F.Cu") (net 5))
 (segment (start 144.85 30.0505) (end 145.127 30.0505) (width 0.2) (layer "F.Cu") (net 5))
 (segment (start 149 40.0505) (end 147.5 40.0505) (width 0.2) (layer "F.Cu") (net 5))
 (segment (start 150.72 29.2705) (end 150 29.2705) (width 0.2) (layer "F.Cu") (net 5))
 (segment (start 149 40.0505) (end 149.026 40.0765) (width 0.2) (layer "F.Cu") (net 5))
 (segment (start 148.98 30.8505) (end 149 30.8305) (width 0.2) (layer "F.Cu") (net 5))
 (segment (start 150.776 29.3265) (end 150.72 29.2705) (width 0.2) (layer "F.Cu") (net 5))
 (segment (start 150.9 32.0505) (end 151.95 32.0505) (width 0.2) (layer "F.Cu") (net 5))
 (segment (start 151.95 32.0505) (end 152 32.0005) (width 0.2) (layer "F.Cu") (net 5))
 (segment (start 150.35 30.3005) (end 150.8 30.7505) (width 0.2) (layer "F.Cu") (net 5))
 (segment (start 151.7 33.6505) (end 152.252 33.6505) (width 0.2) (layer "F.Cu") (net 5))
 (segment (start 145.876 26.9265) (end 145.5 26.5505) (width 0.2) (layer "F.Cu") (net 5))
 (segment (start 150.28 30.3005) (end 150.35 30.3005) (width 0.2) (layer "F.Cu") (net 5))
 (segment (start 152.652 32.6525) (end 152 32.0005) (width 0.2) (layer "F.Cu") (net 5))
 (segment (start 147.475 37.5505) (end 148 37.5505) (width 0.2) (layer "F.Cu") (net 5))
 (segment (start 147.15 30.8505) (end 148.98 30.8505) (width 0.2) (layer "F.Cu") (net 5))
 (segment (start 152 26.6005) (end 151.05 26.6005) (width 0.2) (layer "F.Cu") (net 5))
 (segment (start 145.876 29.3015) (end 145.876 26.9265) (width 0.2) (layer "F.Cu") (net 5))
 (segment (start 146.8 30.8505) (end 147.15 30.8505) (width 0.2) (layer "F.Cu") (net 5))
 (segment (start 152.45 36.5505) (end 152.652 36.3485) (width 0.2) (layer "F.Cu") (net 5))
 (segment (start 145.5 26.5505) (end 145.825 26.5505) (width 0.2) (layer "F.Cu") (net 5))
 (segment (start 146.5 36.5755) (end 147.475 37.5505) (width 0.2) (layer "F.Cu") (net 5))
 (segment (start 150.28 30.3005) (end 150.551262 30.3005) (width 0.2) (layer "F.Cu") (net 5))
 (via (at 149.4 31.7505) (size 0.6) (drill 0.3) (layers "F.Cu" "B.Cu") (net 5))
 (via (at 150.8 30.7505) (size 0.6) (drill 0.3) (layers "F.Cu" "B.Cu") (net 5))
 (via (at 151 26.5505) (size 0.6) (drill 0.3) (layers "F.Cu" "B.Cu") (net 5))
 (via (at 149 40.0505) (size 0.6) (drill 0.3) (layers "F.Cu" "B.Cu") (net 5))
 (via (at 150.9 32.0505) (size 0.6) (drill 0.3) (layers "F.Cu" "B.Cu") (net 5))
 (via (at 145.5 26.5505) (size 0.6) (drill 0.3) (layers "F.Cu" "B.Cu") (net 5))
 (via (at 148 37.5505) (size 0.6) (drill 0.3) (layers "F.Cu" "B.Cu") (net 5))
 (segment (start 148 37.5505) (end 148 39.0505) (width 0.2) (layer "B.Cu") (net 5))
 (segment (start 149.4 31.7505) (end 150.6 31.7505) (width 0.2) (layer "B.Cu") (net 5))
 (segment (start 150.8 31.9505) (end 150.9 32.0505) (width 0.2) (layer "B.Cu") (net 5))
 (segment (start 150.6 31.7505) (end 150.9 32.0505) (width 0.2) (layer "B.Cu") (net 5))
 (segment (start 151 26.5505) (end 145.5 26.5505) (width 0.2) (layer "B.Cu") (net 5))
 (segment (start 148 39.0505) (end 149 40.0505) (width 0.2) (layer "B.Cu") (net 5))
 (segment (start 150.8 30.7505) (end 150.8 31.9505) (width 0.2) (layer "B.Cu") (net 5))
 (segment (start 144.85 30.8505) (end 144.85 32.4005) (width 0.2) (layer "F.Cu") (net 4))
 (segment (start 148 24.600501) (end 148 25.3755) (width 0.2) (layer "F.Cu") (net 4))
 (segment (start 144.85 32.4005) (end 145.087235 32.637735) (width 0.2) (layer "F.Cu") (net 4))
 (segment (start 148 26.6505) (end 148 25.3755) (width 0.2) (layer "F.Cu") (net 4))
 (segment (start 148.7 40.9505) (end 147.6 40.9505) (width 0.2) (layer "F.Cu") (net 4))
 (segment (start 148.3 36.1505) (end 147.575 36.1505) (width 0.2) (layer "F.Cu") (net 4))
 (segment (start 149.5 30.241274) (end 149.414924 30.156198) (width 0.2) (layer "F.Cu") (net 4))
 (segment (start 144.573 30.8505) (end 144.274 30.5515) (width 0.2) (layer "F.Cu") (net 4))
 (segment (start 148.6 27.2505) (end 148 26.6505) (width 0.2) (layer "F.Cu") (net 4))
 (segment (start 144.274 26.684532) (end 146.659032 24.2995) (width 0.2) (layer "F.Cu") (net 4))
 (segment (start 147.698999 24.2995) (end 148 24.600501) (width 0.2) (layer "F.Cu") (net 4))
 (segment (start 147.575 36.1505) (end 147.525 36.2005) (width 0.2) (layer "F.Cu") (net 4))
 (segment (start 144.85 30.8505) (end 144.573 30.8505) (width 0.2) (layer "F.Cu") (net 4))
 (segment (start 146.659032 24.2995) (end 147.698999 24.2995) (width 0.2) (layer "F.Cu") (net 4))
 (segment (start 144.274 30.5515) (end 144.274 26.684532) (width 0.2) (layer "F.Cu") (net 4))
 (segment (start 147.6 40.9505) (end 147.5 41.0505) (width 0.2) (layer "F.Cu") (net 4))
 (segment (start 149.5 30.8305) (end 149.5 30.241274) (width 0.2) (layer "F.Cu") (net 4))
 (via (at 148.6 27.2505) (size 0.6) (drill 0.3) (layers "F.Cu" "B.Cu") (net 4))
 (via (at 148.7 40.9505) (size 0.6) (drill 0.3) (layers "F.Cu" "B.Cu") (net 4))
 (via (at 149.414924 30.156198) (size 0.6) (drill 0.3) (layers "F.Cu" "B.Cu") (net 4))
 (via (at 148.3 36.1505) (size 0.6) (drill 0.3) (layers "F.Cu" "B.Cu") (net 4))
 (via (at 145.087235 32.637735) (size 0.6) (drill 0.3) (layers "F.Cu" "B.Cu") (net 4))
 (segment (start 145.087235 32.637735) (end 145.087235 34.287678) (width 0.2) (layer "B.Cu") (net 4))
 (segment (start 149.6 40.300443) (end 148.949943 40.9505) (width 0.2) (layer "B.Cu") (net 4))
 (segment (start 149.414924 30.156198) (end 149.414924 28.065424) (width 0.2) (layer "B.Cu") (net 4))
 (segment (start 148.3 36.1505) (end 149.6 37.4505) (width 0.2) (layer "B.Cu") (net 4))
 (segment (start 149.414924 28.065424) (end 148.6 27.2505) (width 0.2) (layer "B.Cu") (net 4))
 (segment (start 148.949943 40.9505) (end 148.7 40.9505) (width 0.2) (layer "B.Cu") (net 4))
 (segment (start 145.087235 34.287678) (end 146.950057 36.1505) (width 0.2) (layer "B.Cu") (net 4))
 (segment (start 146.950057 36.1505) (end 148.3 36.1505) (width 0.2) (layer "B.Cu") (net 4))
 (segment (start 149.6 37.4505) (end 149.6 40.300443) (width 0.2) (layer "B.Cu") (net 4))
 (segment (start 149.4 25.7755) (end 149.4 27.8505) (width 0.2) (layer "F.Cu") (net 3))
 (segment (start 145.173 33.9005) (end 145.475 33.9005) (width 0.2) (layer "F.Cu") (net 3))
 (segment (start 144.749 34.3245) (end 145.173 33.9005) (width 0.2) (layer "F.Cu") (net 3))
 (segment (start 149.4 27.8505) (end 148 27.8505) (width 0.2) (layer "F.Cu") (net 3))
 (segment (start 145.5 41.0505) (end 145.35 41.0505) (width 0.2) (layer "F.Cu") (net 3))
 (segment (start 145.475 33.0985) (end 146.923 31.6505) (width 0.2) (layer "F.Cu") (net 3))
 (segment (start 144.749 40.4495) (end 144.749 34.3245) (width 0.2) (layer "F.Cu") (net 3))
 (segment (start 148.448738 30.3005) (end 148.224 30.075762) (width 0.2) (layer "F.Cu") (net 3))
 (segment (start 149 25.3755) (end 149.4 25.7755) (width 0.2) (layer "F.Cu") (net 3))
 (segment (start 148.72 30.3005) (end 148.448738 30.3005) (width 0.2) (layer "F.Cu") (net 3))
 (segment (start 148.224 30.075762) (end 148.224 28.0745) (width 0.2) (layer "F.Cu") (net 3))
 (segment (start 145.35 41.0505) (end 144.749 40.4495) (width 0.2) (layer "F.Cu") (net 3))
 (segment (start 146.923 31.6505) (end 147.8 31.6505) (width 0.2) (layer "F.Cu") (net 3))
 (segment (start 146.968555 28.542585) (end 146.968555 29.069055) (width 0.2) (layer "F.Cu") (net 3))
 (segment (start 148.224 28.0745) (end 148 27.8505) (width 0.2) (layer "F.Cu") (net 3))
 (segment (start 145.475 33.9005) (end 145.475 33.0985) (width 0.2) (layer "F.Cu") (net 3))
 (segment (start 146.968555 29.069055) (end 147.15 29.2505) (width 0.2) (layer "F.Cu") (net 3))
 (via (at 148 27.8505) (size 0.6) (drill 0.3) (layers "F.Cu" "B.Cu") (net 3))
 (via (at 147.8 31.6505) (size 0.6) (drill 0.3) (layers "F.Cu" "B.Cu") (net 3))
 (via (at 146.968555 28.542585) (size 0.6) (drill 0.3) (layers "F.Cu" "B.Cu") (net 3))
 (segment (start 147.8 29.37403) (end 146.968555 28.542585) (width 0.2) (layer "B.Cu") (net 3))
 (segment (start 148 27.8505) (end 147.66064 27.8505) (width 0.2) (layer "B.Cu") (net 3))
 (segment (start 147.66064 27.8505) (end 146.968555 28.542585) (width 0.2) (layer "B.Cu") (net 3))
 (segment (start 147.8 31.6505) (end 147.8 29.37403) (width 0.2) (layer "B.Cu") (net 3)))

